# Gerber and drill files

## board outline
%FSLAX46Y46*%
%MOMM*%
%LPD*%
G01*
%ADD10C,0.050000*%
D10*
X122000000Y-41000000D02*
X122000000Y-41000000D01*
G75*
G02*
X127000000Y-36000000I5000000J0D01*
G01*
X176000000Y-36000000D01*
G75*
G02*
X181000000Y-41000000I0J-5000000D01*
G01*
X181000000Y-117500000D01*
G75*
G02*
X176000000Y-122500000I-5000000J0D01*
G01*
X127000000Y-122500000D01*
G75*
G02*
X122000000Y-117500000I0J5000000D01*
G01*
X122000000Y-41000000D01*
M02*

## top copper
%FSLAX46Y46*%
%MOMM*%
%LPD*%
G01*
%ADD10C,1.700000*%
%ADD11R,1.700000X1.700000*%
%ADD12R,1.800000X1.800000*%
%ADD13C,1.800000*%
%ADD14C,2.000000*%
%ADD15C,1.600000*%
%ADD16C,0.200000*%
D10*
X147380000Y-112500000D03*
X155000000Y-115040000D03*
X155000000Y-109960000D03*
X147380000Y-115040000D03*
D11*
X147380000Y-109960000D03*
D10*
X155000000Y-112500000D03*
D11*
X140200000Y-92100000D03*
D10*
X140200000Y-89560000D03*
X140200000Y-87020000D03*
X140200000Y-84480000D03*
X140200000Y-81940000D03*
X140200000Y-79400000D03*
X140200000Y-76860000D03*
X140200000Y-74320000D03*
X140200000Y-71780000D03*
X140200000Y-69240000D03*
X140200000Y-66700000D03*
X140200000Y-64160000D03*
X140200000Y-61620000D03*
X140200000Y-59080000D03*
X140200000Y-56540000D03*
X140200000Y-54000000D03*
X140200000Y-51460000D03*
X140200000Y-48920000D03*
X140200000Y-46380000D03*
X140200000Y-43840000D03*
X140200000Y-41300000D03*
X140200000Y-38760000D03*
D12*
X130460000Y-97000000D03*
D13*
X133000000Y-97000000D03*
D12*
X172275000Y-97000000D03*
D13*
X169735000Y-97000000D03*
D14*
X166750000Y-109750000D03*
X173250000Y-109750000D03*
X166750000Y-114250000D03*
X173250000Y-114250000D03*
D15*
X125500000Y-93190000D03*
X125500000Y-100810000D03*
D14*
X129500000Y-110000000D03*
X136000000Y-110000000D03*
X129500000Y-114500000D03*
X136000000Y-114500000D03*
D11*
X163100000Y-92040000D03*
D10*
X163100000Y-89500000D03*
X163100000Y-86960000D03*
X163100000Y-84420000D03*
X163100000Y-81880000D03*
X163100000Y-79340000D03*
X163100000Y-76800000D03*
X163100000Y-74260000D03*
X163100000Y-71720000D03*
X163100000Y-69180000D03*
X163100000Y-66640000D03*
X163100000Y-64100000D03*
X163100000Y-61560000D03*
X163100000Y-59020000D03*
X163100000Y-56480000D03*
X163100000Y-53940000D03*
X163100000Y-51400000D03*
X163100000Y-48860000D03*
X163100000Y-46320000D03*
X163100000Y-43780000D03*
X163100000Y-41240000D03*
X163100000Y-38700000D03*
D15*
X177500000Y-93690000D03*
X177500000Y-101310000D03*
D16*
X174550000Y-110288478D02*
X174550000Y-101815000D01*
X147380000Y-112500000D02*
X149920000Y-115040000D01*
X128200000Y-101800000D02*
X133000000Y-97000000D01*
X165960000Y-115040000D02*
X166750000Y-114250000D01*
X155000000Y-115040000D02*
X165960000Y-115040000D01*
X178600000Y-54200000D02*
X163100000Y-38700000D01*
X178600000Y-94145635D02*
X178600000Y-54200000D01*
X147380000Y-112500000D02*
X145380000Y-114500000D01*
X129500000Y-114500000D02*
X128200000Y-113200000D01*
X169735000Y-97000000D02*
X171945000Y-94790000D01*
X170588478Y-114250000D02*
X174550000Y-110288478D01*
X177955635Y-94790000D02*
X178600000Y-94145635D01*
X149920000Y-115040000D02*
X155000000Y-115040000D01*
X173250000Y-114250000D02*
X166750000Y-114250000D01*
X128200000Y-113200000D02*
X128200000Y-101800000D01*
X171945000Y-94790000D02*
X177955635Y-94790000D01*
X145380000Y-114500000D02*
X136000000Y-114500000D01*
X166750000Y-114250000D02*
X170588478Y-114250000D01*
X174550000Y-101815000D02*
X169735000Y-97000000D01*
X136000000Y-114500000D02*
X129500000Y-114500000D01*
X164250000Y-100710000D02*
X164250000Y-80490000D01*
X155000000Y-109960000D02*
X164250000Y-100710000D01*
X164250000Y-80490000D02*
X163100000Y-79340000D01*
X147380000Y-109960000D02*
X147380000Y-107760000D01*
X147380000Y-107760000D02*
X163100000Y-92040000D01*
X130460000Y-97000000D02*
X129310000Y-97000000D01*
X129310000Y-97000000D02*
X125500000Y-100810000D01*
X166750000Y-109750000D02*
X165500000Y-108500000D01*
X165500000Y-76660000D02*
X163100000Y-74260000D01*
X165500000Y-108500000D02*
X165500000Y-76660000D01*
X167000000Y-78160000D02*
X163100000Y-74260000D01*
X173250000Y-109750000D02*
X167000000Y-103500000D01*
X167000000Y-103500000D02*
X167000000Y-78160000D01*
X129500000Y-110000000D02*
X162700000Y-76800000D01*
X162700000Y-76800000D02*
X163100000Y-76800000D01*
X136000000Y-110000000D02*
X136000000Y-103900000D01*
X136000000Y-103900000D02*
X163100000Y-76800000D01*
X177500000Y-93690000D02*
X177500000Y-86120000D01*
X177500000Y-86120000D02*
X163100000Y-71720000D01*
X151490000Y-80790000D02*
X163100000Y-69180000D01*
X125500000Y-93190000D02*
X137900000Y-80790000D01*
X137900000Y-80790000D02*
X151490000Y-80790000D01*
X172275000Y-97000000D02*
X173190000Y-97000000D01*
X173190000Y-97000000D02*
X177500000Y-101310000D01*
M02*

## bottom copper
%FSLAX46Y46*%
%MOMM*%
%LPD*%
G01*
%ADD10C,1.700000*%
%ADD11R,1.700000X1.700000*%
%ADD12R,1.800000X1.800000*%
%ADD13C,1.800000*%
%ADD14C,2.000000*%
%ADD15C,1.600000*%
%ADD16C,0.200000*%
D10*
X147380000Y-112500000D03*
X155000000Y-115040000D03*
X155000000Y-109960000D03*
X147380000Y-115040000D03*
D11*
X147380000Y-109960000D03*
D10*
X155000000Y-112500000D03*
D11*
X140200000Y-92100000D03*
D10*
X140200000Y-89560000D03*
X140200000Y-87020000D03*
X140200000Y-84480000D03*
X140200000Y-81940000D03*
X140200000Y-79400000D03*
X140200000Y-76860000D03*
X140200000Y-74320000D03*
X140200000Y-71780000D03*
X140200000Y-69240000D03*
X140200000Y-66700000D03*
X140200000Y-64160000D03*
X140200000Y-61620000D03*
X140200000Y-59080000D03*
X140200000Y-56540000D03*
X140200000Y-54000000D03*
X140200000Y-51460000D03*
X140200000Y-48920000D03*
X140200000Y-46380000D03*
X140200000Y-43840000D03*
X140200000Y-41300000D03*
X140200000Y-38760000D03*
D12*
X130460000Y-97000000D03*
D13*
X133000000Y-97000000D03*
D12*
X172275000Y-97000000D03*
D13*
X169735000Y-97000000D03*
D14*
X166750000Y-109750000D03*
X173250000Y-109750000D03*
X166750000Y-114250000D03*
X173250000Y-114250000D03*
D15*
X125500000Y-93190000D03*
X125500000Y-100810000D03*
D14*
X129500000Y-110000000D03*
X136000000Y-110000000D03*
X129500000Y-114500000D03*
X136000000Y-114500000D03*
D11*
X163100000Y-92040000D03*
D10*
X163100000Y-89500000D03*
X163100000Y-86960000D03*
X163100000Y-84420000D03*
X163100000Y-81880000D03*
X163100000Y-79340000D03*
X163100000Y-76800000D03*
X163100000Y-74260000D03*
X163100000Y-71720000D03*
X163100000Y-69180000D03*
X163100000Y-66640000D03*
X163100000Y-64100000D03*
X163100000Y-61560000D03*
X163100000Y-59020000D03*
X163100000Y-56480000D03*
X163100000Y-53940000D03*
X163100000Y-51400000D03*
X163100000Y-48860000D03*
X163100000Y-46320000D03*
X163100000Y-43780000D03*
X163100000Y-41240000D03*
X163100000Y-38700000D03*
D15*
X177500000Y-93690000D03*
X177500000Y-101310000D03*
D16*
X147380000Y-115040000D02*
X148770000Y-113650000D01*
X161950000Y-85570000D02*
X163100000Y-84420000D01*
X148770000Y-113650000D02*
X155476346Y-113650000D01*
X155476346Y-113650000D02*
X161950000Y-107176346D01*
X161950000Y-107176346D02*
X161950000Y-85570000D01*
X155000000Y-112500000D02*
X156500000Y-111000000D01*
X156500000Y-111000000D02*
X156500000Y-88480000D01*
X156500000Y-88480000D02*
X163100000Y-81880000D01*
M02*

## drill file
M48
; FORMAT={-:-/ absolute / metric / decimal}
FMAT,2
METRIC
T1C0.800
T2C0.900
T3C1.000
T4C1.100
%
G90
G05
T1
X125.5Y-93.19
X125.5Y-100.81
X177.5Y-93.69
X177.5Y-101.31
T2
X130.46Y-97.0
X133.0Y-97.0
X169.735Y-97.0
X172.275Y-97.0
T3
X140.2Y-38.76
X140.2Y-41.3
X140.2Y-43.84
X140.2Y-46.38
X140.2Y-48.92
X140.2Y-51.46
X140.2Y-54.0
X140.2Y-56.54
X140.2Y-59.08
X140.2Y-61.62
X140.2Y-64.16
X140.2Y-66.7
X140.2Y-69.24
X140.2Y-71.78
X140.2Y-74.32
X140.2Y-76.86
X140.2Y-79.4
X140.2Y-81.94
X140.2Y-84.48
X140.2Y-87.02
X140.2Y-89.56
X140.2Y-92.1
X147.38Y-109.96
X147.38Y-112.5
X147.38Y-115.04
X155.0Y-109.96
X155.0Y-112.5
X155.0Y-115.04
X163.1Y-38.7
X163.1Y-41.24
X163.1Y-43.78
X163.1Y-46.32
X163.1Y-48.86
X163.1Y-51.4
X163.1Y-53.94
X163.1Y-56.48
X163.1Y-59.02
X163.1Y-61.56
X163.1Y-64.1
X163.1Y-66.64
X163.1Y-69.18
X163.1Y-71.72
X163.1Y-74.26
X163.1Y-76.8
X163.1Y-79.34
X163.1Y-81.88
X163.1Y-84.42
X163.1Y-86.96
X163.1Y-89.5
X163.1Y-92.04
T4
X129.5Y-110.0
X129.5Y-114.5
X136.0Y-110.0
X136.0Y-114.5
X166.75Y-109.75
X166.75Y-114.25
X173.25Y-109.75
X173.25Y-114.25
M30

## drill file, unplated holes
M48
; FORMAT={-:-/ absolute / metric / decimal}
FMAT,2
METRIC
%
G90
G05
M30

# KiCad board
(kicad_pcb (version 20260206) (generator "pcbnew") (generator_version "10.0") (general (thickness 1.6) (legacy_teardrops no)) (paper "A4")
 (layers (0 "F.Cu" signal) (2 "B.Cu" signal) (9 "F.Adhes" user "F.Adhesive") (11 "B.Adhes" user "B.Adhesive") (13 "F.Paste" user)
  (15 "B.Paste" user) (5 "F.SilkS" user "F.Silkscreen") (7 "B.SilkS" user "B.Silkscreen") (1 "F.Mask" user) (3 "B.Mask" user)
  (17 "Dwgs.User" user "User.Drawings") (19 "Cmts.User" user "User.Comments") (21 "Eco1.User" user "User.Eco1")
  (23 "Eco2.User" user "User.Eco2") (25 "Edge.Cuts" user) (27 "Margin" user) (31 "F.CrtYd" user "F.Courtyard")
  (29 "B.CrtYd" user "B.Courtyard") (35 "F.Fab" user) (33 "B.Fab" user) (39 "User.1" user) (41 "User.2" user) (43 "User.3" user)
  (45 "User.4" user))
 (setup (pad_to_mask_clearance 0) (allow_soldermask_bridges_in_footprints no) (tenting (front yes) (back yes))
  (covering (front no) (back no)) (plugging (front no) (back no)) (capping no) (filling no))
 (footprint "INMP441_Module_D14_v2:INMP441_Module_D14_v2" (layer "F.Cu") (at 151.19 112.5)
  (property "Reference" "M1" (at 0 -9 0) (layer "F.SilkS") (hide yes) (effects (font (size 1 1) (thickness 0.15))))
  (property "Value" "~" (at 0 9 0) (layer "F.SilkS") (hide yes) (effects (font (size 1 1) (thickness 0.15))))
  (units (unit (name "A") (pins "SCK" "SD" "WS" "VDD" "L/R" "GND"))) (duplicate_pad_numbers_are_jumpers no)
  (pad "GND" thru_hole circle (at -3.81 0) (size 1.7 1.7) (drill 1) (layers "*.Cu" "*.Mask" "F.SilkS") (remove_unused_layers no) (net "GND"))
  (pad "L/R" thru_hole circle (at 3.81 2.54) (size 1.7 1.7) (drill 1) (layers "*.Cu" "*.Mask" "F.SilkS") (remove_unused_layers no)
   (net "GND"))
  (pad "SCK" thru_hole circle (at 3.81 -2.54) (size 1.7 1.7) (drill 1) (layers "*.Cu" "*.Mask" "F.SilkS") (remove_unused_layers no)
   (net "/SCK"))
  (pad "SD" thru_hole circle (at -3.81 2.54) (size 1.7 1.7) (drill 1) (layers "*.Cu" "*.Mask" "F.SilkS") (remove_unused_layers no)
   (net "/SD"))
  (pad "VDD" thru_hole rect (at -3.81 -2.54) (size 1.7 1.7) (drill 1) (layers "*.Cu" "*.Mask" "F.SilkS") (remove_unused_layers no)
   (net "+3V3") (thermal_bridge_angle 45))
  (pad "WS" thru_hole circle (at 3.81 0) (size 1.7 1.7) (drill 1) (layers "*.Cu" "*.Mask" "F.SilkS") (remove_unused_layers no) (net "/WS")))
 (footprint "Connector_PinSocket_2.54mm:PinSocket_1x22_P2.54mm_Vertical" (layer "F.Cu") (at 140.2 92.1 180)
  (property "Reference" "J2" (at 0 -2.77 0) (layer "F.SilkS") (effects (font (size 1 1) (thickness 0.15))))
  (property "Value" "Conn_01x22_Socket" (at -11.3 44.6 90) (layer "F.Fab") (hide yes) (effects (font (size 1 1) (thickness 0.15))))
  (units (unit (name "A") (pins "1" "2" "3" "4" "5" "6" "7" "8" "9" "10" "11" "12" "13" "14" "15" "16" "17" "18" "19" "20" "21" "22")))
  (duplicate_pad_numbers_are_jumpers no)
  (pad "1" thru_hole rect (at 0 0 180) (size 1.7 1.7) (drill 1) (layers "*.Cu" "*.Mask") (remove_unused_layers no)
   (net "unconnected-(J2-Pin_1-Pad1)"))
  (pad "2" thru_hole circle (at 0 2.54 180) (size 1.7 1.7) (drill 1) (layers "*.Cu" "*.Mask") (remove_unused_layers no)
   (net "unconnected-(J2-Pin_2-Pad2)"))
  (pad "3" thru_hole circle (at 0 5.08 180) (size 1.7 1.7) (drill 1) (layers "*.Cu" "*.Mask") (remove_unused_layers no)
   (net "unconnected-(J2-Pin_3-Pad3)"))
  (pad "4" thru_hole circle (at 0 7.62 180) (size 1.7 1.7) (drill 1) (layers "*.Cu" "*.Mask") (remove_unused_layers no)
   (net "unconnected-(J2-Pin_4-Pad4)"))
  (pad "5" thru_hole circle (at 0 10.16 180) (size 1.7 1.7) (drill 1) (layers "*.Cu" "*.Mask") (remove_unused_layers no)
   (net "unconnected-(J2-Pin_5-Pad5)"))
  (pad "6" thru_hole circle (at 0 12.7 180) (size 1.7 1.7) (drill 1) (layers "*.Cu" "*.Mask") (remove_unused_layers no)
   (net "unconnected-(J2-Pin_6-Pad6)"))
  (pad "7" thru_hole circle (at 0 15.24 180) (size 1.7 1.7) (drill 1) (layers "*.Cu" "*.Mask") (remove_unused_layers no)
   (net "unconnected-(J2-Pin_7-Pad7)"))
  (pad "8" thru_hole circle (at 0 17.78 180) (size 1.7 1.7) (drill 1) (layers "*.Cu" "*.Mask") (remove_unused_layers no)
   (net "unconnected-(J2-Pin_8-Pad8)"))
  (pad "9" thru_hole circle (at 0 20.32 180) (size 1.7 1.7) (drill 1) (layers "*.Cu" "*.Mask") (remove_unused_layers no)
   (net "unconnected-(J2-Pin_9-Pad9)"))
  (pad "10" thru_hole circle (at 0 22.86 180) (size 1.7 1.7) (drill 1) (layers "*.Cu" "*.Mask") (remove_unused_layers no)
   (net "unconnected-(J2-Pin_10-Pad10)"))
  (pad "11" thru_hole circle (at 0 25.4 180) (size 1.7 1.7) (drill 1) (layers "*.Cu" "*.Mask") (remove_unused_layers no)
   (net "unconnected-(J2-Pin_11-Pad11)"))
  (pad "12" thru_hole circle (at 0 27.94 180) (size 1.7 1.7) (drill 1) (layers "*.Cu" "*.Mask") (remove_unused_layers no)
   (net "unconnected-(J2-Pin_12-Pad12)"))
  (pad "13" thru_hole circle (at 0 30.48 180) (size 1.7 1.7) (drill 1) (layers "*.Cu" "*.Mask") (remove_unused_layers no)
   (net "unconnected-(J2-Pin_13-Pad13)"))
  (pad "14" thru_hole circle (at 0 33.02 180) (size 1.7 1.7) (drill 1) (layers "*.Cu" "*.Mask") (remove_unused_layers no)
   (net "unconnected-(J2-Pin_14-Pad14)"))
  (pad "15" thru_hole circle (at 0 35.56 180) (size 1.7 1.7) (drill 1) (layers "*.Cu" "*.Mask") (remove_unused_layers no)
   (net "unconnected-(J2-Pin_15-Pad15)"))
  (pad "16" thru_hole circle (at 0 38.1 180) (size 1.7 1.7) (drill 1) (layers "*.Cu" "*.Mask") (remove_unused_layers no)
   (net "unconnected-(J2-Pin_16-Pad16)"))
  (pad "17" thru_hole circle (at 0 40.64 180) (size 1.7 1.7) (drill 1) (layers "*.Cu" "*.Mask") (remove_unused_layers no)
   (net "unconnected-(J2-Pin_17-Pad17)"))
  (pad "18" thru_hole circle (at 0 43.18 180) (size 1.7 1.7) (drill 1) (layers "*.Cu" "*.Mask") (remove_unused_layers no)
   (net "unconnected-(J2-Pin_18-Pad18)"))
  (pad "19" thru_hole circle (at 0 45.72 180) (size 1.7 1.7) (drill 1) (layers "*.Cu" "*.Mask") (remove_unused_layers no)
   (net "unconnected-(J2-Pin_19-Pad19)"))
  (pad "20" thru_hole circle (at 0 48.26 180) (size 1.7 1.7) (drill 1) (layers "*.Cu" "*.Mask") (remove_unused_layers no)
   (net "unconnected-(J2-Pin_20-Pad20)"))
  (pad "21" thru_hole circle (at 0 50.8 180) (size 1.7 1.7) (drill 1) (layers "*.Cu" "*.Mask") (remove_unused_layers no)
   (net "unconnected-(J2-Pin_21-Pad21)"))
  (pad "22" thru_hole circle (at 0 53.34 180) (size 1.7 1.7) (drill 1) (layers "*.Cu" "*.Mask") (remove_unused_layers no)
   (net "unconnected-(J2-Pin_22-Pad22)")))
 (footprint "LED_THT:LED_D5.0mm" (layer "F.Cu") (at 130.46 97)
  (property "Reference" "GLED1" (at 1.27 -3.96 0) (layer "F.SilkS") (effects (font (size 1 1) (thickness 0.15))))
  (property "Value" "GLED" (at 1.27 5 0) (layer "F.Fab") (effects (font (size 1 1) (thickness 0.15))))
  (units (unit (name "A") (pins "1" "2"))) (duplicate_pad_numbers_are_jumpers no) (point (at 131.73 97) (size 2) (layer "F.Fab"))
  (pad "1" thru_hole rect (at 0 0) (size 1.8 1.8) (drill 0.9) (layers "*.Cu" "*.Mask") (remove_unused_layers no) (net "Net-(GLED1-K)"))
  (pad "2" thru_hole circle (at 2.54 0) (size 1.8 1.8) (drill 0.9) (layers "*.Cu" "*.Mask") (remove_unused_layers no) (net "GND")))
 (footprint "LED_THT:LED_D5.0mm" (layer "F.Cu") (at 172.275 97 180)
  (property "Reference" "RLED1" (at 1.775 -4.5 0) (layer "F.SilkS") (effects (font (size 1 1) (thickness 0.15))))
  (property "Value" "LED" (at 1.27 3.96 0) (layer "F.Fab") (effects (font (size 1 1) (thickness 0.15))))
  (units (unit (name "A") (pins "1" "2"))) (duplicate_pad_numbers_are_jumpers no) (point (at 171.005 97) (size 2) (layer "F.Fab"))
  (pad "1" thru_hole rect (at 0 0 180) (size 1.8 1.8) (drill 0.9) (layers "*.Cu" "*.Mask") (remove_unused_layers no) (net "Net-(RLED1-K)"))
  (pad "2" thru_hole circle (at 2.54 0 180) (size 1.8 1.8) (drill 0.9) (layers "*.Cu" "*.Mask") (remove_unused_layers no) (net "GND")))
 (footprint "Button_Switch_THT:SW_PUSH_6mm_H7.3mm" (layer "F.Cu") (at 166.75 109.75)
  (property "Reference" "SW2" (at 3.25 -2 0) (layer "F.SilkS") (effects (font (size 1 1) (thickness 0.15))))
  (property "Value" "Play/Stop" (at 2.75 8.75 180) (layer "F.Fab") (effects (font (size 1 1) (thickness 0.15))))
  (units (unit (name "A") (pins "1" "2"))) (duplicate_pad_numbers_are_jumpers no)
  (pad "1" thru_hole circle (at 0 0 90) (size 2 2) (drill 1.1) (layers "*.Cu" "*.Mask") (remove_unused_layers no)
   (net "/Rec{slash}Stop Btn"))
  (pad "1" thru_hole circle (at 6.5 0 90) (size 2 2) (drill 1.1) (layers "*.Cu" "*.Mask") (remove_unused_layers no)
   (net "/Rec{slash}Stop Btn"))
  (pad "2" thru_hole circle (at 0 4.5 90) (size 2 2) (drill 1.1) (layers "*.Cu" "*.Mask") (remove_unused_layers no) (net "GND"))
  (pad "2" thru_hole circle (at 6.5 4.5 90) (size 2 2) (drill 1.1) (layers "*.Cu" "*.Mask") (remove_unused_layers no) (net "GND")))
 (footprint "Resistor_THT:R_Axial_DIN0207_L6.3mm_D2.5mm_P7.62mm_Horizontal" (layer "F.Cu") (at 125.5 93.19 -90)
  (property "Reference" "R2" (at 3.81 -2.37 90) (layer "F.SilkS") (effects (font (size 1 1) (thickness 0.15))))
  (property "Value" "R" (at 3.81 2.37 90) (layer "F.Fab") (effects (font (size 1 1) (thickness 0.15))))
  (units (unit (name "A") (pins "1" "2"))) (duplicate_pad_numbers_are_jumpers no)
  (pad "1" thru_hole circle (at 0 0 270) (size 1.6 1.6) (drill 0.8) (layers "*.Cu" "*.Mask") (remove_unused_layers no) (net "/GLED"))
  (pad "2" thru_hole circle (at 7.62 0 270) (size 1.6 1.6) (drill 0.8) (layers "*.Cu" "*.Mask") (remove_unused_layers no)
   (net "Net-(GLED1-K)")))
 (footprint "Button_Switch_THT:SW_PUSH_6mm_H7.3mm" (layer "F.Cu") (at 129.5 110)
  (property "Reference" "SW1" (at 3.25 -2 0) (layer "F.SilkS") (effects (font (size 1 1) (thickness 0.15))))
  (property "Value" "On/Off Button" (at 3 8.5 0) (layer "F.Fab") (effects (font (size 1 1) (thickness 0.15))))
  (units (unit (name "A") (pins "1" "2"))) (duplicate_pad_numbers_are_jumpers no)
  (pad "1" thru_hole circle (at 0 0 90) (size 2 2) (drill 1.1) (layers "*.Cu" "*.Mask") (remove_unused_layers no) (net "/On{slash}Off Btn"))
  (pad "1" thru_hole circle (at 6.5 0 90) (size 2 2) (drill 1.1) (layers "*.Cu" "*.Mask") (remove_unused_layers no)
   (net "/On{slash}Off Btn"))
  (pad "2" thru_hole circle (at 0 4.5 90) (size 2 2) (drill 1.1) (layers "*.Cu" "*.Mask") (remove_unused_layers no) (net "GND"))
  (pad "2" thru_hole circle (at 6.5 4.5 90) (size 2 2) (drill 1.1) (layers "*.Cu" "*.Mask") (remove_unused_layers no) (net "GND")))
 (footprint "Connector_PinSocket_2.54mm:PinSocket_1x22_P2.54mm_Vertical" (layer "F.Cu") (at 163.1 92.04 180)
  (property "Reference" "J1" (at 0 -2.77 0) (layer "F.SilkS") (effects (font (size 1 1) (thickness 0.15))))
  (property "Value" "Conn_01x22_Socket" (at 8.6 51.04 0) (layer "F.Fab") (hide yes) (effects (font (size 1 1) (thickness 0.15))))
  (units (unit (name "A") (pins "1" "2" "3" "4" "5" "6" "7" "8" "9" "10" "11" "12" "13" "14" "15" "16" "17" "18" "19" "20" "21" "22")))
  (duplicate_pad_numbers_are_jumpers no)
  (pad "1" thru_hole rect (at 0 0 180) (size 1.7 1.7) (drill 1) (layers "*.Cu" "*.Mask") (remove_unused_layers no) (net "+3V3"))
  (pad "2" thru_hole circle (at 0 2.54 180) (size 1.7 1.7) (drill 1) (layers "*.Cu" "*.Mask") (remove_unused_layers no)
   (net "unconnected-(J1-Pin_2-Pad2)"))
  (pad "3" thru_hole circle (at 0 5.08 180) (size 1.7 1.7) (drill 1) (layers "*.Cu" "*.Mask") (remove_unused_layers no)
   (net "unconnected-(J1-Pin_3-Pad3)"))
  (pad "4" thru_hole circle (at 0 7.62 180) (size 1.7 1.7) (drill 1) (layers "*.Cu" "*.Mask") (remove_unused_layers no) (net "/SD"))
  (pad "5" thru_hole circle (at 0 10.16 180) (size 1.7 1.7) (drill 1) (layers "*.Cu" "*.Mask") (remove_unused_layers no) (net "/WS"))
  (pad "6" thru_hole circle (at 0 12.7 180) (size 1.7 1.7) (drill 1) (layers "*.Cu" "*.Mask") (remove_unused_layers no) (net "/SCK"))
  (pad "7" thru_hole circle (at 0 15.24 180) (size 1.7 1.7) (drill 1) (layers "*.Cu" "*.Mask") (remove_unused_layers no)
   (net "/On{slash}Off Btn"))
  (pad "8" thru_hole circle (at 0 17.78 180) (size 1.7 1.7) (drill 1) (layers "*.Cu" "*.Mask") (remove_unused_layers no)
   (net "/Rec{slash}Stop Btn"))
  (pad "9" thru_hole circle (at 0 20.32 180) (size 1.7 1.7) (drill 1) (layers "*.Cu" "*.Mask") (remove_unused_layers no) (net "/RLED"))
  (pad "10" thru_hole circle (at 0 22.86 180) (size 1.7 1.7) (drill 1) (layers "*.Cu" "*.Mask") (remove_unused_layers no) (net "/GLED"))
  (pad "11" thru_hole circle (at 0 25.4 180) (size 1.7 1.7) (drill 1) (layers "*.Cu" "*.Mask") (remove_unused_layers no)
   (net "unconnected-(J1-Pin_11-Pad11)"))
  (pad "12" thru_hole circle (at 0 27.94 180) (size 1.7 1.7) (drill 1) (layers "*.Cu" "*.Mask") (remove_unused_layers no)
   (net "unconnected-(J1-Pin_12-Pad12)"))
  (pad "13" thru_hole circle (at 0 30.48 180) (size 1.7 1.7) (drill 1) (layers "*.Cu" "*.Mask") (remove_unused_layers no)
   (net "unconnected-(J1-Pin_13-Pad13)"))
  (pad "14" thru_hole circle (at 0 33.02 180) (size 1.7 1.7) (drill 1) (layers "*.Cu" "*.Mask") (remove_unused_layers no)
   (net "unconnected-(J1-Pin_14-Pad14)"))
  (pad "15" thru_hole circle (at 0 35.56 180) (size 1.7 1.7) (drill 1) (layers "*.Cu" "*.Mask") (remove_unused_layers no)
   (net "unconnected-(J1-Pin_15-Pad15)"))
  (pad "16" thru_hole circle (at 0 38.1 180) (size 1.7 1.7) (drill 1) (layers "*.Cu" "*.Mask") (remove_unused_layers no)
   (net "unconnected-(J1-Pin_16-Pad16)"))
  (pad "17" thru_hole circle (at 0 40.64 180) (size 1.7 1.7) (drill 1) (layers "*.Cu" "*.Mask") (remove_unused_layers no)
   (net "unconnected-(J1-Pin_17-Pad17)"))
  (pad "18" thru_hole circle (at 0 43.18 180) (size 1.7 1.7) (drill 1) (layers "*.Cu" "*.Mask") (remove_unused_layers no)
   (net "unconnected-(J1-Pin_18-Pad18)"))
  (pad "19" thru_hole circle (at 0 45.72 180) (size 1.7 1.7) (drill 1) (layers "*.Cu" "*.Mask") (remove_unused_layers no)
   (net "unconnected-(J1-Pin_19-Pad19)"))
  (pad "20" thru_hole circle (at 0 48.26 180) (size 1.7 1.7) (drill 1) (layers "*.Cu" "*.Mask") (remove_unused_layers no)
   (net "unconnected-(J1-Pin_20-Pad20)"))
  (pad "21" thru_hole circle (at 0 50.8 180) (size 1.7 1.7) (drill 1) (layers "*.Cu" "*.Mask") (remove_unused_layers no)
   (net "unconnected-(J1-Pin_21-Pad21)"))
  (pad "22" thru_hole circle (at 0 53.34 180) (size 1.7 1.7) (drill 1) (layers "*.Cu" "*.Mask") (remove_unused_layers no) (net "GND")))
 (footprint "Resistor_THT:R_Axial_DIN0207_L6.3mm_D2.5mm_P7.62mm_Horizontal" (layer "F.Cu") (at 177.5 93.69 -90)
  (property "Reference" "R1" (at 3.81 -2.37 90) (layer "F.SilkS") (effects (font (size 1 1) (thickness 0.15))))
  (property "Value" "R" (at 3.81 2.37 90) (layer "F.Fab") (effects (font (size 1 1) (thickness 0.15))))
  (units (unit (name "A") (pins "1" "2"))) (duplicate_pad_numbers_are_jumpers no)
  (pad "1" thru_hole circle (at 0 0 270) (size 1.6 1.6) (drill 0.8) (layers "*.Cu" "*.Mask") (remove_unused_layers no) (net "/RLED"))
  (pad "2" thru_hole circle (at 7.62 0 270) (size 1.6 1.6) (drill 0.8) (layers "*.Cu" "*.Mask") (remove_unused_layers no)
   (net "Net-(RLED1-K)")))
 (gr_rect (start 122 36) (end 181 122.5) (radius 5) (stroke (width 0.05) (type solid)) (fill no) (layer "Edge.Cuts"))
 (segment (start 174.55 110.288478) (end 174.55 101.815) (width 0.2) (layer "F.Cu") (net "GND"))
 (segment (start 147.38 112.5) (end 149.92 115.04) (width 0.2) (layer "F.Cu") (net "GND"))
 (segment (start 128.2 101.8) (end 133 97) (width 0.2) (layer "F.Cu") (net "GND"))
 (segment (start 165.96 115.04) (end 166.75 114.25) (width 0.2) (layer "F.Cu") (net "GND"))
 (segment (start 155 115.04) (end 165.96 115.04) (width 0.2) (layer "F.Cu") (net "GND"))
 (segment (start 178.6 54.2) (end 163.1 38.7) (width 0.2) (layer "F.Cu") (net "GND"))
 (segment (start 178.6 94.145635) (end 178.6 54.2) (width 0.2) (layer "F.Cu") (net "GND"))
 (segment (start 147.38 112.5) (end 145.38 114.5) (width 0.2) (layer "F.Cu") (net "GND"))
 (segment (start 129.5 114.5) (end 128.2 113.2) (width 0.2) (layer "F.Cu") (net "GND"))
 (segment (start 169.735 97) (end 171.945 94.79) (width 0.2) (layer "F.Cu") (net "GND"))
 (segment (start 170.588478 114.25) (end 174.55 110.288478) (width 0.2) (layer "F.Cu") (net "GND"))
 (segment (start 177.955635 94.79) (end 178.6 94.145635) (width 0.2) (layer "F.Cu") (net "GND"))
 (segment (start 149.92 115.04) (end 155 115.04) (width 0.2) (layer "F.Cu") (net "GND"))
 (segment (start 173.25 114.25) (end 166.75 114.25) (width 0.2) (layer "F.Cu") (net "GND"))
 (segment (start 128.2 113.2) (end 128.2 101.8) (width 0.2) (layer "F.Cu") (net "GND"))
 (segment (start 171.945 94.79) (end 177.955635 94.79) (width 0.2) (layer "F.Cu") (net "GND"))
 (segment (start 145.38 114.5) (end 136 114.5) (width 0.2) (layer "F.Cu") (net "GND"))
 (segment (start 166.75 114.25) (end 170.588478 114.25) (width 0.2) (layer "F.Cu") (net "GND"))
 (segment (start 174.55 101.815) (end 169.735 97) (width 0.2) (layer "F.Cu") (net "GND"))
 (segment (start 136 114.5) (end 129.5 114.5) (width 0.2) (layer "F.Cu") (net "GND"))
 (segment (start 164.25 100.71) (end 164.25 80.49) (width 0.2) (layer "F.Cu") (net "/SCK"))
 (segment (start 155 109.96) (end 164.25 100.71) (width 0.2) (layer "F.Cu") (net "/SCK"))
 (segment (start 164.25 80.49) (end 163.1 79.34) (width 0.2) (layer "F.Cu") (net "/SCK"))
 (segment (start 147.38 115.04) (end 148.77 113.65) (width 0.2) (layer "B.Cu") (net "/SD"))
 (segment (start 161.95 85.57) (end 163.1 84.42) (width 0.2) (layer "B.Cu") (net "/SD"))
 (segment (start 148.77 113.65) (end 155.476346 113.65) (width 0.2) (layer "B.Cu") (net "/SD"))
 (segment (start 155.476346 113.65) (end 161.95 107.176346) (width 0.2) (layer "B.Cu") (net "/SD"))
 (segment (start 161.95 107.176346) (end 161.95 85.57) (width 0.2) (layer "B.Cu") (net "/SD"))
 (segment (start 147.38 109.96) (end 147.38 107.76) (width 0.2) (layer "F.Cu") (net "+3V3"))
 (segment (start 147.38 107.76) (end 163.1 92.04) (width 0.2) (layer "F.Cu") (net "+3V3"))
 (segment (start 155 112.5) (end 156.5 111) (width 0.2) (layer "B.Cu") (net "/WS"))
 (segment (start 156.5 111) (end 156.5 88.48) (width 0.2) (layer "B.Cu") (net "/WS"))
 (segment (start 156.5 88.48) (end 163.1 81.88) (width 0.2) (layer "B.Cu") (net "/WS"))
 (segment (start 130.46 97) (end 129.31 97) (width 0.2) (layer "F.Cu") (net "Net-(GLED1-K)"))
 (segment (start 129.31 97) (end 125.5 100.81) (width 0.2) (layer "F.Cu") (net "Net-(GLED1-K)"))
 (segment (start 166.75 109.75) (end 165.5 108.5) (width 0.2) (layer "F.Cu") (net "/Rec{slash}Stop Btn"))
 (segment (start 165.5 76.66) (end 163.1 74.26) (width 0.2) (layer "F.Cu") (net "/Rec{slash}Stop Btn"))
 (segment (start 165.5 108.5) (end 165.5 76.66) (width 0.2) (layer "F.Cu") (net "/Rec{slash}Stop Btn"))
 (segment (start 167 78.16) (end 163.1 74.26) (width 0.2) (layer "F.Cu") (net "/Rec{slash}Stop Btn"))
 (segment (start 173.25 109.75) (end 167 103.5) (width 0.2) (layer "F.Cu") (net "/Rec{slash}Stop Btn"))
 (segment (start 167 103.5) (end 167 78.16) (width 0.2) (layer "F.Cu") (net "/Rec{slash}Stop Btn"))
 (segment (start 129.5 110) (end 162.7 76.8) (width 0.2) (layer "F.Cu") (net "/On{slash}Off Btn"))
 (segment (start 162.7 76.8) (end 163.1 76.8) (width 0.2) (layer "F.Cu") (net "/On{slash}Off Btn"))
 (segment (start 136 110) (end 136 103.9) (width 0.2) (layer "F.Cu") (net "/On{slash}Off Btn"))
 (segment (start 136 103.9) (end 163.1 76.8) (width 0.2) (layer "F.Cu") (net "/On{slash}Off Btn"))
 (segment (start 177.5 93.69) (end 177.5 86.12) (width 0.2) (layer "F.Cu") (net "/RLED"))
 (segment (start 177.5 86.12) (end 163.1 71.72) (width 0.2) (layer "F.Cu") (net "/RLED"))
 (segment (start 151.49 80.79) (end 163.1 69.18) (width 0.2) (layer "F.Cu") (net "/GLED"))
 (segment (start 125.5 93.19) (end 137.9 80.79) (width 0.2) (layer "F.Cu") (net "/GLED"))
 (segment (start 137.9 80.79) (end 151.49 80.79) (width 0.2) (layer "F.Cu") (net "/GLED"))
 (segment (start 172.275 97) (end 173.19 97) (width 0.2) (layer "F.Cu") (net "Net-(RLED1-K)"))
 (segment (start 173.19 97) (end 177.5 101.31) (width 0.2) (layer "F.Cu") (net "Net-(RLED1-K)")))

